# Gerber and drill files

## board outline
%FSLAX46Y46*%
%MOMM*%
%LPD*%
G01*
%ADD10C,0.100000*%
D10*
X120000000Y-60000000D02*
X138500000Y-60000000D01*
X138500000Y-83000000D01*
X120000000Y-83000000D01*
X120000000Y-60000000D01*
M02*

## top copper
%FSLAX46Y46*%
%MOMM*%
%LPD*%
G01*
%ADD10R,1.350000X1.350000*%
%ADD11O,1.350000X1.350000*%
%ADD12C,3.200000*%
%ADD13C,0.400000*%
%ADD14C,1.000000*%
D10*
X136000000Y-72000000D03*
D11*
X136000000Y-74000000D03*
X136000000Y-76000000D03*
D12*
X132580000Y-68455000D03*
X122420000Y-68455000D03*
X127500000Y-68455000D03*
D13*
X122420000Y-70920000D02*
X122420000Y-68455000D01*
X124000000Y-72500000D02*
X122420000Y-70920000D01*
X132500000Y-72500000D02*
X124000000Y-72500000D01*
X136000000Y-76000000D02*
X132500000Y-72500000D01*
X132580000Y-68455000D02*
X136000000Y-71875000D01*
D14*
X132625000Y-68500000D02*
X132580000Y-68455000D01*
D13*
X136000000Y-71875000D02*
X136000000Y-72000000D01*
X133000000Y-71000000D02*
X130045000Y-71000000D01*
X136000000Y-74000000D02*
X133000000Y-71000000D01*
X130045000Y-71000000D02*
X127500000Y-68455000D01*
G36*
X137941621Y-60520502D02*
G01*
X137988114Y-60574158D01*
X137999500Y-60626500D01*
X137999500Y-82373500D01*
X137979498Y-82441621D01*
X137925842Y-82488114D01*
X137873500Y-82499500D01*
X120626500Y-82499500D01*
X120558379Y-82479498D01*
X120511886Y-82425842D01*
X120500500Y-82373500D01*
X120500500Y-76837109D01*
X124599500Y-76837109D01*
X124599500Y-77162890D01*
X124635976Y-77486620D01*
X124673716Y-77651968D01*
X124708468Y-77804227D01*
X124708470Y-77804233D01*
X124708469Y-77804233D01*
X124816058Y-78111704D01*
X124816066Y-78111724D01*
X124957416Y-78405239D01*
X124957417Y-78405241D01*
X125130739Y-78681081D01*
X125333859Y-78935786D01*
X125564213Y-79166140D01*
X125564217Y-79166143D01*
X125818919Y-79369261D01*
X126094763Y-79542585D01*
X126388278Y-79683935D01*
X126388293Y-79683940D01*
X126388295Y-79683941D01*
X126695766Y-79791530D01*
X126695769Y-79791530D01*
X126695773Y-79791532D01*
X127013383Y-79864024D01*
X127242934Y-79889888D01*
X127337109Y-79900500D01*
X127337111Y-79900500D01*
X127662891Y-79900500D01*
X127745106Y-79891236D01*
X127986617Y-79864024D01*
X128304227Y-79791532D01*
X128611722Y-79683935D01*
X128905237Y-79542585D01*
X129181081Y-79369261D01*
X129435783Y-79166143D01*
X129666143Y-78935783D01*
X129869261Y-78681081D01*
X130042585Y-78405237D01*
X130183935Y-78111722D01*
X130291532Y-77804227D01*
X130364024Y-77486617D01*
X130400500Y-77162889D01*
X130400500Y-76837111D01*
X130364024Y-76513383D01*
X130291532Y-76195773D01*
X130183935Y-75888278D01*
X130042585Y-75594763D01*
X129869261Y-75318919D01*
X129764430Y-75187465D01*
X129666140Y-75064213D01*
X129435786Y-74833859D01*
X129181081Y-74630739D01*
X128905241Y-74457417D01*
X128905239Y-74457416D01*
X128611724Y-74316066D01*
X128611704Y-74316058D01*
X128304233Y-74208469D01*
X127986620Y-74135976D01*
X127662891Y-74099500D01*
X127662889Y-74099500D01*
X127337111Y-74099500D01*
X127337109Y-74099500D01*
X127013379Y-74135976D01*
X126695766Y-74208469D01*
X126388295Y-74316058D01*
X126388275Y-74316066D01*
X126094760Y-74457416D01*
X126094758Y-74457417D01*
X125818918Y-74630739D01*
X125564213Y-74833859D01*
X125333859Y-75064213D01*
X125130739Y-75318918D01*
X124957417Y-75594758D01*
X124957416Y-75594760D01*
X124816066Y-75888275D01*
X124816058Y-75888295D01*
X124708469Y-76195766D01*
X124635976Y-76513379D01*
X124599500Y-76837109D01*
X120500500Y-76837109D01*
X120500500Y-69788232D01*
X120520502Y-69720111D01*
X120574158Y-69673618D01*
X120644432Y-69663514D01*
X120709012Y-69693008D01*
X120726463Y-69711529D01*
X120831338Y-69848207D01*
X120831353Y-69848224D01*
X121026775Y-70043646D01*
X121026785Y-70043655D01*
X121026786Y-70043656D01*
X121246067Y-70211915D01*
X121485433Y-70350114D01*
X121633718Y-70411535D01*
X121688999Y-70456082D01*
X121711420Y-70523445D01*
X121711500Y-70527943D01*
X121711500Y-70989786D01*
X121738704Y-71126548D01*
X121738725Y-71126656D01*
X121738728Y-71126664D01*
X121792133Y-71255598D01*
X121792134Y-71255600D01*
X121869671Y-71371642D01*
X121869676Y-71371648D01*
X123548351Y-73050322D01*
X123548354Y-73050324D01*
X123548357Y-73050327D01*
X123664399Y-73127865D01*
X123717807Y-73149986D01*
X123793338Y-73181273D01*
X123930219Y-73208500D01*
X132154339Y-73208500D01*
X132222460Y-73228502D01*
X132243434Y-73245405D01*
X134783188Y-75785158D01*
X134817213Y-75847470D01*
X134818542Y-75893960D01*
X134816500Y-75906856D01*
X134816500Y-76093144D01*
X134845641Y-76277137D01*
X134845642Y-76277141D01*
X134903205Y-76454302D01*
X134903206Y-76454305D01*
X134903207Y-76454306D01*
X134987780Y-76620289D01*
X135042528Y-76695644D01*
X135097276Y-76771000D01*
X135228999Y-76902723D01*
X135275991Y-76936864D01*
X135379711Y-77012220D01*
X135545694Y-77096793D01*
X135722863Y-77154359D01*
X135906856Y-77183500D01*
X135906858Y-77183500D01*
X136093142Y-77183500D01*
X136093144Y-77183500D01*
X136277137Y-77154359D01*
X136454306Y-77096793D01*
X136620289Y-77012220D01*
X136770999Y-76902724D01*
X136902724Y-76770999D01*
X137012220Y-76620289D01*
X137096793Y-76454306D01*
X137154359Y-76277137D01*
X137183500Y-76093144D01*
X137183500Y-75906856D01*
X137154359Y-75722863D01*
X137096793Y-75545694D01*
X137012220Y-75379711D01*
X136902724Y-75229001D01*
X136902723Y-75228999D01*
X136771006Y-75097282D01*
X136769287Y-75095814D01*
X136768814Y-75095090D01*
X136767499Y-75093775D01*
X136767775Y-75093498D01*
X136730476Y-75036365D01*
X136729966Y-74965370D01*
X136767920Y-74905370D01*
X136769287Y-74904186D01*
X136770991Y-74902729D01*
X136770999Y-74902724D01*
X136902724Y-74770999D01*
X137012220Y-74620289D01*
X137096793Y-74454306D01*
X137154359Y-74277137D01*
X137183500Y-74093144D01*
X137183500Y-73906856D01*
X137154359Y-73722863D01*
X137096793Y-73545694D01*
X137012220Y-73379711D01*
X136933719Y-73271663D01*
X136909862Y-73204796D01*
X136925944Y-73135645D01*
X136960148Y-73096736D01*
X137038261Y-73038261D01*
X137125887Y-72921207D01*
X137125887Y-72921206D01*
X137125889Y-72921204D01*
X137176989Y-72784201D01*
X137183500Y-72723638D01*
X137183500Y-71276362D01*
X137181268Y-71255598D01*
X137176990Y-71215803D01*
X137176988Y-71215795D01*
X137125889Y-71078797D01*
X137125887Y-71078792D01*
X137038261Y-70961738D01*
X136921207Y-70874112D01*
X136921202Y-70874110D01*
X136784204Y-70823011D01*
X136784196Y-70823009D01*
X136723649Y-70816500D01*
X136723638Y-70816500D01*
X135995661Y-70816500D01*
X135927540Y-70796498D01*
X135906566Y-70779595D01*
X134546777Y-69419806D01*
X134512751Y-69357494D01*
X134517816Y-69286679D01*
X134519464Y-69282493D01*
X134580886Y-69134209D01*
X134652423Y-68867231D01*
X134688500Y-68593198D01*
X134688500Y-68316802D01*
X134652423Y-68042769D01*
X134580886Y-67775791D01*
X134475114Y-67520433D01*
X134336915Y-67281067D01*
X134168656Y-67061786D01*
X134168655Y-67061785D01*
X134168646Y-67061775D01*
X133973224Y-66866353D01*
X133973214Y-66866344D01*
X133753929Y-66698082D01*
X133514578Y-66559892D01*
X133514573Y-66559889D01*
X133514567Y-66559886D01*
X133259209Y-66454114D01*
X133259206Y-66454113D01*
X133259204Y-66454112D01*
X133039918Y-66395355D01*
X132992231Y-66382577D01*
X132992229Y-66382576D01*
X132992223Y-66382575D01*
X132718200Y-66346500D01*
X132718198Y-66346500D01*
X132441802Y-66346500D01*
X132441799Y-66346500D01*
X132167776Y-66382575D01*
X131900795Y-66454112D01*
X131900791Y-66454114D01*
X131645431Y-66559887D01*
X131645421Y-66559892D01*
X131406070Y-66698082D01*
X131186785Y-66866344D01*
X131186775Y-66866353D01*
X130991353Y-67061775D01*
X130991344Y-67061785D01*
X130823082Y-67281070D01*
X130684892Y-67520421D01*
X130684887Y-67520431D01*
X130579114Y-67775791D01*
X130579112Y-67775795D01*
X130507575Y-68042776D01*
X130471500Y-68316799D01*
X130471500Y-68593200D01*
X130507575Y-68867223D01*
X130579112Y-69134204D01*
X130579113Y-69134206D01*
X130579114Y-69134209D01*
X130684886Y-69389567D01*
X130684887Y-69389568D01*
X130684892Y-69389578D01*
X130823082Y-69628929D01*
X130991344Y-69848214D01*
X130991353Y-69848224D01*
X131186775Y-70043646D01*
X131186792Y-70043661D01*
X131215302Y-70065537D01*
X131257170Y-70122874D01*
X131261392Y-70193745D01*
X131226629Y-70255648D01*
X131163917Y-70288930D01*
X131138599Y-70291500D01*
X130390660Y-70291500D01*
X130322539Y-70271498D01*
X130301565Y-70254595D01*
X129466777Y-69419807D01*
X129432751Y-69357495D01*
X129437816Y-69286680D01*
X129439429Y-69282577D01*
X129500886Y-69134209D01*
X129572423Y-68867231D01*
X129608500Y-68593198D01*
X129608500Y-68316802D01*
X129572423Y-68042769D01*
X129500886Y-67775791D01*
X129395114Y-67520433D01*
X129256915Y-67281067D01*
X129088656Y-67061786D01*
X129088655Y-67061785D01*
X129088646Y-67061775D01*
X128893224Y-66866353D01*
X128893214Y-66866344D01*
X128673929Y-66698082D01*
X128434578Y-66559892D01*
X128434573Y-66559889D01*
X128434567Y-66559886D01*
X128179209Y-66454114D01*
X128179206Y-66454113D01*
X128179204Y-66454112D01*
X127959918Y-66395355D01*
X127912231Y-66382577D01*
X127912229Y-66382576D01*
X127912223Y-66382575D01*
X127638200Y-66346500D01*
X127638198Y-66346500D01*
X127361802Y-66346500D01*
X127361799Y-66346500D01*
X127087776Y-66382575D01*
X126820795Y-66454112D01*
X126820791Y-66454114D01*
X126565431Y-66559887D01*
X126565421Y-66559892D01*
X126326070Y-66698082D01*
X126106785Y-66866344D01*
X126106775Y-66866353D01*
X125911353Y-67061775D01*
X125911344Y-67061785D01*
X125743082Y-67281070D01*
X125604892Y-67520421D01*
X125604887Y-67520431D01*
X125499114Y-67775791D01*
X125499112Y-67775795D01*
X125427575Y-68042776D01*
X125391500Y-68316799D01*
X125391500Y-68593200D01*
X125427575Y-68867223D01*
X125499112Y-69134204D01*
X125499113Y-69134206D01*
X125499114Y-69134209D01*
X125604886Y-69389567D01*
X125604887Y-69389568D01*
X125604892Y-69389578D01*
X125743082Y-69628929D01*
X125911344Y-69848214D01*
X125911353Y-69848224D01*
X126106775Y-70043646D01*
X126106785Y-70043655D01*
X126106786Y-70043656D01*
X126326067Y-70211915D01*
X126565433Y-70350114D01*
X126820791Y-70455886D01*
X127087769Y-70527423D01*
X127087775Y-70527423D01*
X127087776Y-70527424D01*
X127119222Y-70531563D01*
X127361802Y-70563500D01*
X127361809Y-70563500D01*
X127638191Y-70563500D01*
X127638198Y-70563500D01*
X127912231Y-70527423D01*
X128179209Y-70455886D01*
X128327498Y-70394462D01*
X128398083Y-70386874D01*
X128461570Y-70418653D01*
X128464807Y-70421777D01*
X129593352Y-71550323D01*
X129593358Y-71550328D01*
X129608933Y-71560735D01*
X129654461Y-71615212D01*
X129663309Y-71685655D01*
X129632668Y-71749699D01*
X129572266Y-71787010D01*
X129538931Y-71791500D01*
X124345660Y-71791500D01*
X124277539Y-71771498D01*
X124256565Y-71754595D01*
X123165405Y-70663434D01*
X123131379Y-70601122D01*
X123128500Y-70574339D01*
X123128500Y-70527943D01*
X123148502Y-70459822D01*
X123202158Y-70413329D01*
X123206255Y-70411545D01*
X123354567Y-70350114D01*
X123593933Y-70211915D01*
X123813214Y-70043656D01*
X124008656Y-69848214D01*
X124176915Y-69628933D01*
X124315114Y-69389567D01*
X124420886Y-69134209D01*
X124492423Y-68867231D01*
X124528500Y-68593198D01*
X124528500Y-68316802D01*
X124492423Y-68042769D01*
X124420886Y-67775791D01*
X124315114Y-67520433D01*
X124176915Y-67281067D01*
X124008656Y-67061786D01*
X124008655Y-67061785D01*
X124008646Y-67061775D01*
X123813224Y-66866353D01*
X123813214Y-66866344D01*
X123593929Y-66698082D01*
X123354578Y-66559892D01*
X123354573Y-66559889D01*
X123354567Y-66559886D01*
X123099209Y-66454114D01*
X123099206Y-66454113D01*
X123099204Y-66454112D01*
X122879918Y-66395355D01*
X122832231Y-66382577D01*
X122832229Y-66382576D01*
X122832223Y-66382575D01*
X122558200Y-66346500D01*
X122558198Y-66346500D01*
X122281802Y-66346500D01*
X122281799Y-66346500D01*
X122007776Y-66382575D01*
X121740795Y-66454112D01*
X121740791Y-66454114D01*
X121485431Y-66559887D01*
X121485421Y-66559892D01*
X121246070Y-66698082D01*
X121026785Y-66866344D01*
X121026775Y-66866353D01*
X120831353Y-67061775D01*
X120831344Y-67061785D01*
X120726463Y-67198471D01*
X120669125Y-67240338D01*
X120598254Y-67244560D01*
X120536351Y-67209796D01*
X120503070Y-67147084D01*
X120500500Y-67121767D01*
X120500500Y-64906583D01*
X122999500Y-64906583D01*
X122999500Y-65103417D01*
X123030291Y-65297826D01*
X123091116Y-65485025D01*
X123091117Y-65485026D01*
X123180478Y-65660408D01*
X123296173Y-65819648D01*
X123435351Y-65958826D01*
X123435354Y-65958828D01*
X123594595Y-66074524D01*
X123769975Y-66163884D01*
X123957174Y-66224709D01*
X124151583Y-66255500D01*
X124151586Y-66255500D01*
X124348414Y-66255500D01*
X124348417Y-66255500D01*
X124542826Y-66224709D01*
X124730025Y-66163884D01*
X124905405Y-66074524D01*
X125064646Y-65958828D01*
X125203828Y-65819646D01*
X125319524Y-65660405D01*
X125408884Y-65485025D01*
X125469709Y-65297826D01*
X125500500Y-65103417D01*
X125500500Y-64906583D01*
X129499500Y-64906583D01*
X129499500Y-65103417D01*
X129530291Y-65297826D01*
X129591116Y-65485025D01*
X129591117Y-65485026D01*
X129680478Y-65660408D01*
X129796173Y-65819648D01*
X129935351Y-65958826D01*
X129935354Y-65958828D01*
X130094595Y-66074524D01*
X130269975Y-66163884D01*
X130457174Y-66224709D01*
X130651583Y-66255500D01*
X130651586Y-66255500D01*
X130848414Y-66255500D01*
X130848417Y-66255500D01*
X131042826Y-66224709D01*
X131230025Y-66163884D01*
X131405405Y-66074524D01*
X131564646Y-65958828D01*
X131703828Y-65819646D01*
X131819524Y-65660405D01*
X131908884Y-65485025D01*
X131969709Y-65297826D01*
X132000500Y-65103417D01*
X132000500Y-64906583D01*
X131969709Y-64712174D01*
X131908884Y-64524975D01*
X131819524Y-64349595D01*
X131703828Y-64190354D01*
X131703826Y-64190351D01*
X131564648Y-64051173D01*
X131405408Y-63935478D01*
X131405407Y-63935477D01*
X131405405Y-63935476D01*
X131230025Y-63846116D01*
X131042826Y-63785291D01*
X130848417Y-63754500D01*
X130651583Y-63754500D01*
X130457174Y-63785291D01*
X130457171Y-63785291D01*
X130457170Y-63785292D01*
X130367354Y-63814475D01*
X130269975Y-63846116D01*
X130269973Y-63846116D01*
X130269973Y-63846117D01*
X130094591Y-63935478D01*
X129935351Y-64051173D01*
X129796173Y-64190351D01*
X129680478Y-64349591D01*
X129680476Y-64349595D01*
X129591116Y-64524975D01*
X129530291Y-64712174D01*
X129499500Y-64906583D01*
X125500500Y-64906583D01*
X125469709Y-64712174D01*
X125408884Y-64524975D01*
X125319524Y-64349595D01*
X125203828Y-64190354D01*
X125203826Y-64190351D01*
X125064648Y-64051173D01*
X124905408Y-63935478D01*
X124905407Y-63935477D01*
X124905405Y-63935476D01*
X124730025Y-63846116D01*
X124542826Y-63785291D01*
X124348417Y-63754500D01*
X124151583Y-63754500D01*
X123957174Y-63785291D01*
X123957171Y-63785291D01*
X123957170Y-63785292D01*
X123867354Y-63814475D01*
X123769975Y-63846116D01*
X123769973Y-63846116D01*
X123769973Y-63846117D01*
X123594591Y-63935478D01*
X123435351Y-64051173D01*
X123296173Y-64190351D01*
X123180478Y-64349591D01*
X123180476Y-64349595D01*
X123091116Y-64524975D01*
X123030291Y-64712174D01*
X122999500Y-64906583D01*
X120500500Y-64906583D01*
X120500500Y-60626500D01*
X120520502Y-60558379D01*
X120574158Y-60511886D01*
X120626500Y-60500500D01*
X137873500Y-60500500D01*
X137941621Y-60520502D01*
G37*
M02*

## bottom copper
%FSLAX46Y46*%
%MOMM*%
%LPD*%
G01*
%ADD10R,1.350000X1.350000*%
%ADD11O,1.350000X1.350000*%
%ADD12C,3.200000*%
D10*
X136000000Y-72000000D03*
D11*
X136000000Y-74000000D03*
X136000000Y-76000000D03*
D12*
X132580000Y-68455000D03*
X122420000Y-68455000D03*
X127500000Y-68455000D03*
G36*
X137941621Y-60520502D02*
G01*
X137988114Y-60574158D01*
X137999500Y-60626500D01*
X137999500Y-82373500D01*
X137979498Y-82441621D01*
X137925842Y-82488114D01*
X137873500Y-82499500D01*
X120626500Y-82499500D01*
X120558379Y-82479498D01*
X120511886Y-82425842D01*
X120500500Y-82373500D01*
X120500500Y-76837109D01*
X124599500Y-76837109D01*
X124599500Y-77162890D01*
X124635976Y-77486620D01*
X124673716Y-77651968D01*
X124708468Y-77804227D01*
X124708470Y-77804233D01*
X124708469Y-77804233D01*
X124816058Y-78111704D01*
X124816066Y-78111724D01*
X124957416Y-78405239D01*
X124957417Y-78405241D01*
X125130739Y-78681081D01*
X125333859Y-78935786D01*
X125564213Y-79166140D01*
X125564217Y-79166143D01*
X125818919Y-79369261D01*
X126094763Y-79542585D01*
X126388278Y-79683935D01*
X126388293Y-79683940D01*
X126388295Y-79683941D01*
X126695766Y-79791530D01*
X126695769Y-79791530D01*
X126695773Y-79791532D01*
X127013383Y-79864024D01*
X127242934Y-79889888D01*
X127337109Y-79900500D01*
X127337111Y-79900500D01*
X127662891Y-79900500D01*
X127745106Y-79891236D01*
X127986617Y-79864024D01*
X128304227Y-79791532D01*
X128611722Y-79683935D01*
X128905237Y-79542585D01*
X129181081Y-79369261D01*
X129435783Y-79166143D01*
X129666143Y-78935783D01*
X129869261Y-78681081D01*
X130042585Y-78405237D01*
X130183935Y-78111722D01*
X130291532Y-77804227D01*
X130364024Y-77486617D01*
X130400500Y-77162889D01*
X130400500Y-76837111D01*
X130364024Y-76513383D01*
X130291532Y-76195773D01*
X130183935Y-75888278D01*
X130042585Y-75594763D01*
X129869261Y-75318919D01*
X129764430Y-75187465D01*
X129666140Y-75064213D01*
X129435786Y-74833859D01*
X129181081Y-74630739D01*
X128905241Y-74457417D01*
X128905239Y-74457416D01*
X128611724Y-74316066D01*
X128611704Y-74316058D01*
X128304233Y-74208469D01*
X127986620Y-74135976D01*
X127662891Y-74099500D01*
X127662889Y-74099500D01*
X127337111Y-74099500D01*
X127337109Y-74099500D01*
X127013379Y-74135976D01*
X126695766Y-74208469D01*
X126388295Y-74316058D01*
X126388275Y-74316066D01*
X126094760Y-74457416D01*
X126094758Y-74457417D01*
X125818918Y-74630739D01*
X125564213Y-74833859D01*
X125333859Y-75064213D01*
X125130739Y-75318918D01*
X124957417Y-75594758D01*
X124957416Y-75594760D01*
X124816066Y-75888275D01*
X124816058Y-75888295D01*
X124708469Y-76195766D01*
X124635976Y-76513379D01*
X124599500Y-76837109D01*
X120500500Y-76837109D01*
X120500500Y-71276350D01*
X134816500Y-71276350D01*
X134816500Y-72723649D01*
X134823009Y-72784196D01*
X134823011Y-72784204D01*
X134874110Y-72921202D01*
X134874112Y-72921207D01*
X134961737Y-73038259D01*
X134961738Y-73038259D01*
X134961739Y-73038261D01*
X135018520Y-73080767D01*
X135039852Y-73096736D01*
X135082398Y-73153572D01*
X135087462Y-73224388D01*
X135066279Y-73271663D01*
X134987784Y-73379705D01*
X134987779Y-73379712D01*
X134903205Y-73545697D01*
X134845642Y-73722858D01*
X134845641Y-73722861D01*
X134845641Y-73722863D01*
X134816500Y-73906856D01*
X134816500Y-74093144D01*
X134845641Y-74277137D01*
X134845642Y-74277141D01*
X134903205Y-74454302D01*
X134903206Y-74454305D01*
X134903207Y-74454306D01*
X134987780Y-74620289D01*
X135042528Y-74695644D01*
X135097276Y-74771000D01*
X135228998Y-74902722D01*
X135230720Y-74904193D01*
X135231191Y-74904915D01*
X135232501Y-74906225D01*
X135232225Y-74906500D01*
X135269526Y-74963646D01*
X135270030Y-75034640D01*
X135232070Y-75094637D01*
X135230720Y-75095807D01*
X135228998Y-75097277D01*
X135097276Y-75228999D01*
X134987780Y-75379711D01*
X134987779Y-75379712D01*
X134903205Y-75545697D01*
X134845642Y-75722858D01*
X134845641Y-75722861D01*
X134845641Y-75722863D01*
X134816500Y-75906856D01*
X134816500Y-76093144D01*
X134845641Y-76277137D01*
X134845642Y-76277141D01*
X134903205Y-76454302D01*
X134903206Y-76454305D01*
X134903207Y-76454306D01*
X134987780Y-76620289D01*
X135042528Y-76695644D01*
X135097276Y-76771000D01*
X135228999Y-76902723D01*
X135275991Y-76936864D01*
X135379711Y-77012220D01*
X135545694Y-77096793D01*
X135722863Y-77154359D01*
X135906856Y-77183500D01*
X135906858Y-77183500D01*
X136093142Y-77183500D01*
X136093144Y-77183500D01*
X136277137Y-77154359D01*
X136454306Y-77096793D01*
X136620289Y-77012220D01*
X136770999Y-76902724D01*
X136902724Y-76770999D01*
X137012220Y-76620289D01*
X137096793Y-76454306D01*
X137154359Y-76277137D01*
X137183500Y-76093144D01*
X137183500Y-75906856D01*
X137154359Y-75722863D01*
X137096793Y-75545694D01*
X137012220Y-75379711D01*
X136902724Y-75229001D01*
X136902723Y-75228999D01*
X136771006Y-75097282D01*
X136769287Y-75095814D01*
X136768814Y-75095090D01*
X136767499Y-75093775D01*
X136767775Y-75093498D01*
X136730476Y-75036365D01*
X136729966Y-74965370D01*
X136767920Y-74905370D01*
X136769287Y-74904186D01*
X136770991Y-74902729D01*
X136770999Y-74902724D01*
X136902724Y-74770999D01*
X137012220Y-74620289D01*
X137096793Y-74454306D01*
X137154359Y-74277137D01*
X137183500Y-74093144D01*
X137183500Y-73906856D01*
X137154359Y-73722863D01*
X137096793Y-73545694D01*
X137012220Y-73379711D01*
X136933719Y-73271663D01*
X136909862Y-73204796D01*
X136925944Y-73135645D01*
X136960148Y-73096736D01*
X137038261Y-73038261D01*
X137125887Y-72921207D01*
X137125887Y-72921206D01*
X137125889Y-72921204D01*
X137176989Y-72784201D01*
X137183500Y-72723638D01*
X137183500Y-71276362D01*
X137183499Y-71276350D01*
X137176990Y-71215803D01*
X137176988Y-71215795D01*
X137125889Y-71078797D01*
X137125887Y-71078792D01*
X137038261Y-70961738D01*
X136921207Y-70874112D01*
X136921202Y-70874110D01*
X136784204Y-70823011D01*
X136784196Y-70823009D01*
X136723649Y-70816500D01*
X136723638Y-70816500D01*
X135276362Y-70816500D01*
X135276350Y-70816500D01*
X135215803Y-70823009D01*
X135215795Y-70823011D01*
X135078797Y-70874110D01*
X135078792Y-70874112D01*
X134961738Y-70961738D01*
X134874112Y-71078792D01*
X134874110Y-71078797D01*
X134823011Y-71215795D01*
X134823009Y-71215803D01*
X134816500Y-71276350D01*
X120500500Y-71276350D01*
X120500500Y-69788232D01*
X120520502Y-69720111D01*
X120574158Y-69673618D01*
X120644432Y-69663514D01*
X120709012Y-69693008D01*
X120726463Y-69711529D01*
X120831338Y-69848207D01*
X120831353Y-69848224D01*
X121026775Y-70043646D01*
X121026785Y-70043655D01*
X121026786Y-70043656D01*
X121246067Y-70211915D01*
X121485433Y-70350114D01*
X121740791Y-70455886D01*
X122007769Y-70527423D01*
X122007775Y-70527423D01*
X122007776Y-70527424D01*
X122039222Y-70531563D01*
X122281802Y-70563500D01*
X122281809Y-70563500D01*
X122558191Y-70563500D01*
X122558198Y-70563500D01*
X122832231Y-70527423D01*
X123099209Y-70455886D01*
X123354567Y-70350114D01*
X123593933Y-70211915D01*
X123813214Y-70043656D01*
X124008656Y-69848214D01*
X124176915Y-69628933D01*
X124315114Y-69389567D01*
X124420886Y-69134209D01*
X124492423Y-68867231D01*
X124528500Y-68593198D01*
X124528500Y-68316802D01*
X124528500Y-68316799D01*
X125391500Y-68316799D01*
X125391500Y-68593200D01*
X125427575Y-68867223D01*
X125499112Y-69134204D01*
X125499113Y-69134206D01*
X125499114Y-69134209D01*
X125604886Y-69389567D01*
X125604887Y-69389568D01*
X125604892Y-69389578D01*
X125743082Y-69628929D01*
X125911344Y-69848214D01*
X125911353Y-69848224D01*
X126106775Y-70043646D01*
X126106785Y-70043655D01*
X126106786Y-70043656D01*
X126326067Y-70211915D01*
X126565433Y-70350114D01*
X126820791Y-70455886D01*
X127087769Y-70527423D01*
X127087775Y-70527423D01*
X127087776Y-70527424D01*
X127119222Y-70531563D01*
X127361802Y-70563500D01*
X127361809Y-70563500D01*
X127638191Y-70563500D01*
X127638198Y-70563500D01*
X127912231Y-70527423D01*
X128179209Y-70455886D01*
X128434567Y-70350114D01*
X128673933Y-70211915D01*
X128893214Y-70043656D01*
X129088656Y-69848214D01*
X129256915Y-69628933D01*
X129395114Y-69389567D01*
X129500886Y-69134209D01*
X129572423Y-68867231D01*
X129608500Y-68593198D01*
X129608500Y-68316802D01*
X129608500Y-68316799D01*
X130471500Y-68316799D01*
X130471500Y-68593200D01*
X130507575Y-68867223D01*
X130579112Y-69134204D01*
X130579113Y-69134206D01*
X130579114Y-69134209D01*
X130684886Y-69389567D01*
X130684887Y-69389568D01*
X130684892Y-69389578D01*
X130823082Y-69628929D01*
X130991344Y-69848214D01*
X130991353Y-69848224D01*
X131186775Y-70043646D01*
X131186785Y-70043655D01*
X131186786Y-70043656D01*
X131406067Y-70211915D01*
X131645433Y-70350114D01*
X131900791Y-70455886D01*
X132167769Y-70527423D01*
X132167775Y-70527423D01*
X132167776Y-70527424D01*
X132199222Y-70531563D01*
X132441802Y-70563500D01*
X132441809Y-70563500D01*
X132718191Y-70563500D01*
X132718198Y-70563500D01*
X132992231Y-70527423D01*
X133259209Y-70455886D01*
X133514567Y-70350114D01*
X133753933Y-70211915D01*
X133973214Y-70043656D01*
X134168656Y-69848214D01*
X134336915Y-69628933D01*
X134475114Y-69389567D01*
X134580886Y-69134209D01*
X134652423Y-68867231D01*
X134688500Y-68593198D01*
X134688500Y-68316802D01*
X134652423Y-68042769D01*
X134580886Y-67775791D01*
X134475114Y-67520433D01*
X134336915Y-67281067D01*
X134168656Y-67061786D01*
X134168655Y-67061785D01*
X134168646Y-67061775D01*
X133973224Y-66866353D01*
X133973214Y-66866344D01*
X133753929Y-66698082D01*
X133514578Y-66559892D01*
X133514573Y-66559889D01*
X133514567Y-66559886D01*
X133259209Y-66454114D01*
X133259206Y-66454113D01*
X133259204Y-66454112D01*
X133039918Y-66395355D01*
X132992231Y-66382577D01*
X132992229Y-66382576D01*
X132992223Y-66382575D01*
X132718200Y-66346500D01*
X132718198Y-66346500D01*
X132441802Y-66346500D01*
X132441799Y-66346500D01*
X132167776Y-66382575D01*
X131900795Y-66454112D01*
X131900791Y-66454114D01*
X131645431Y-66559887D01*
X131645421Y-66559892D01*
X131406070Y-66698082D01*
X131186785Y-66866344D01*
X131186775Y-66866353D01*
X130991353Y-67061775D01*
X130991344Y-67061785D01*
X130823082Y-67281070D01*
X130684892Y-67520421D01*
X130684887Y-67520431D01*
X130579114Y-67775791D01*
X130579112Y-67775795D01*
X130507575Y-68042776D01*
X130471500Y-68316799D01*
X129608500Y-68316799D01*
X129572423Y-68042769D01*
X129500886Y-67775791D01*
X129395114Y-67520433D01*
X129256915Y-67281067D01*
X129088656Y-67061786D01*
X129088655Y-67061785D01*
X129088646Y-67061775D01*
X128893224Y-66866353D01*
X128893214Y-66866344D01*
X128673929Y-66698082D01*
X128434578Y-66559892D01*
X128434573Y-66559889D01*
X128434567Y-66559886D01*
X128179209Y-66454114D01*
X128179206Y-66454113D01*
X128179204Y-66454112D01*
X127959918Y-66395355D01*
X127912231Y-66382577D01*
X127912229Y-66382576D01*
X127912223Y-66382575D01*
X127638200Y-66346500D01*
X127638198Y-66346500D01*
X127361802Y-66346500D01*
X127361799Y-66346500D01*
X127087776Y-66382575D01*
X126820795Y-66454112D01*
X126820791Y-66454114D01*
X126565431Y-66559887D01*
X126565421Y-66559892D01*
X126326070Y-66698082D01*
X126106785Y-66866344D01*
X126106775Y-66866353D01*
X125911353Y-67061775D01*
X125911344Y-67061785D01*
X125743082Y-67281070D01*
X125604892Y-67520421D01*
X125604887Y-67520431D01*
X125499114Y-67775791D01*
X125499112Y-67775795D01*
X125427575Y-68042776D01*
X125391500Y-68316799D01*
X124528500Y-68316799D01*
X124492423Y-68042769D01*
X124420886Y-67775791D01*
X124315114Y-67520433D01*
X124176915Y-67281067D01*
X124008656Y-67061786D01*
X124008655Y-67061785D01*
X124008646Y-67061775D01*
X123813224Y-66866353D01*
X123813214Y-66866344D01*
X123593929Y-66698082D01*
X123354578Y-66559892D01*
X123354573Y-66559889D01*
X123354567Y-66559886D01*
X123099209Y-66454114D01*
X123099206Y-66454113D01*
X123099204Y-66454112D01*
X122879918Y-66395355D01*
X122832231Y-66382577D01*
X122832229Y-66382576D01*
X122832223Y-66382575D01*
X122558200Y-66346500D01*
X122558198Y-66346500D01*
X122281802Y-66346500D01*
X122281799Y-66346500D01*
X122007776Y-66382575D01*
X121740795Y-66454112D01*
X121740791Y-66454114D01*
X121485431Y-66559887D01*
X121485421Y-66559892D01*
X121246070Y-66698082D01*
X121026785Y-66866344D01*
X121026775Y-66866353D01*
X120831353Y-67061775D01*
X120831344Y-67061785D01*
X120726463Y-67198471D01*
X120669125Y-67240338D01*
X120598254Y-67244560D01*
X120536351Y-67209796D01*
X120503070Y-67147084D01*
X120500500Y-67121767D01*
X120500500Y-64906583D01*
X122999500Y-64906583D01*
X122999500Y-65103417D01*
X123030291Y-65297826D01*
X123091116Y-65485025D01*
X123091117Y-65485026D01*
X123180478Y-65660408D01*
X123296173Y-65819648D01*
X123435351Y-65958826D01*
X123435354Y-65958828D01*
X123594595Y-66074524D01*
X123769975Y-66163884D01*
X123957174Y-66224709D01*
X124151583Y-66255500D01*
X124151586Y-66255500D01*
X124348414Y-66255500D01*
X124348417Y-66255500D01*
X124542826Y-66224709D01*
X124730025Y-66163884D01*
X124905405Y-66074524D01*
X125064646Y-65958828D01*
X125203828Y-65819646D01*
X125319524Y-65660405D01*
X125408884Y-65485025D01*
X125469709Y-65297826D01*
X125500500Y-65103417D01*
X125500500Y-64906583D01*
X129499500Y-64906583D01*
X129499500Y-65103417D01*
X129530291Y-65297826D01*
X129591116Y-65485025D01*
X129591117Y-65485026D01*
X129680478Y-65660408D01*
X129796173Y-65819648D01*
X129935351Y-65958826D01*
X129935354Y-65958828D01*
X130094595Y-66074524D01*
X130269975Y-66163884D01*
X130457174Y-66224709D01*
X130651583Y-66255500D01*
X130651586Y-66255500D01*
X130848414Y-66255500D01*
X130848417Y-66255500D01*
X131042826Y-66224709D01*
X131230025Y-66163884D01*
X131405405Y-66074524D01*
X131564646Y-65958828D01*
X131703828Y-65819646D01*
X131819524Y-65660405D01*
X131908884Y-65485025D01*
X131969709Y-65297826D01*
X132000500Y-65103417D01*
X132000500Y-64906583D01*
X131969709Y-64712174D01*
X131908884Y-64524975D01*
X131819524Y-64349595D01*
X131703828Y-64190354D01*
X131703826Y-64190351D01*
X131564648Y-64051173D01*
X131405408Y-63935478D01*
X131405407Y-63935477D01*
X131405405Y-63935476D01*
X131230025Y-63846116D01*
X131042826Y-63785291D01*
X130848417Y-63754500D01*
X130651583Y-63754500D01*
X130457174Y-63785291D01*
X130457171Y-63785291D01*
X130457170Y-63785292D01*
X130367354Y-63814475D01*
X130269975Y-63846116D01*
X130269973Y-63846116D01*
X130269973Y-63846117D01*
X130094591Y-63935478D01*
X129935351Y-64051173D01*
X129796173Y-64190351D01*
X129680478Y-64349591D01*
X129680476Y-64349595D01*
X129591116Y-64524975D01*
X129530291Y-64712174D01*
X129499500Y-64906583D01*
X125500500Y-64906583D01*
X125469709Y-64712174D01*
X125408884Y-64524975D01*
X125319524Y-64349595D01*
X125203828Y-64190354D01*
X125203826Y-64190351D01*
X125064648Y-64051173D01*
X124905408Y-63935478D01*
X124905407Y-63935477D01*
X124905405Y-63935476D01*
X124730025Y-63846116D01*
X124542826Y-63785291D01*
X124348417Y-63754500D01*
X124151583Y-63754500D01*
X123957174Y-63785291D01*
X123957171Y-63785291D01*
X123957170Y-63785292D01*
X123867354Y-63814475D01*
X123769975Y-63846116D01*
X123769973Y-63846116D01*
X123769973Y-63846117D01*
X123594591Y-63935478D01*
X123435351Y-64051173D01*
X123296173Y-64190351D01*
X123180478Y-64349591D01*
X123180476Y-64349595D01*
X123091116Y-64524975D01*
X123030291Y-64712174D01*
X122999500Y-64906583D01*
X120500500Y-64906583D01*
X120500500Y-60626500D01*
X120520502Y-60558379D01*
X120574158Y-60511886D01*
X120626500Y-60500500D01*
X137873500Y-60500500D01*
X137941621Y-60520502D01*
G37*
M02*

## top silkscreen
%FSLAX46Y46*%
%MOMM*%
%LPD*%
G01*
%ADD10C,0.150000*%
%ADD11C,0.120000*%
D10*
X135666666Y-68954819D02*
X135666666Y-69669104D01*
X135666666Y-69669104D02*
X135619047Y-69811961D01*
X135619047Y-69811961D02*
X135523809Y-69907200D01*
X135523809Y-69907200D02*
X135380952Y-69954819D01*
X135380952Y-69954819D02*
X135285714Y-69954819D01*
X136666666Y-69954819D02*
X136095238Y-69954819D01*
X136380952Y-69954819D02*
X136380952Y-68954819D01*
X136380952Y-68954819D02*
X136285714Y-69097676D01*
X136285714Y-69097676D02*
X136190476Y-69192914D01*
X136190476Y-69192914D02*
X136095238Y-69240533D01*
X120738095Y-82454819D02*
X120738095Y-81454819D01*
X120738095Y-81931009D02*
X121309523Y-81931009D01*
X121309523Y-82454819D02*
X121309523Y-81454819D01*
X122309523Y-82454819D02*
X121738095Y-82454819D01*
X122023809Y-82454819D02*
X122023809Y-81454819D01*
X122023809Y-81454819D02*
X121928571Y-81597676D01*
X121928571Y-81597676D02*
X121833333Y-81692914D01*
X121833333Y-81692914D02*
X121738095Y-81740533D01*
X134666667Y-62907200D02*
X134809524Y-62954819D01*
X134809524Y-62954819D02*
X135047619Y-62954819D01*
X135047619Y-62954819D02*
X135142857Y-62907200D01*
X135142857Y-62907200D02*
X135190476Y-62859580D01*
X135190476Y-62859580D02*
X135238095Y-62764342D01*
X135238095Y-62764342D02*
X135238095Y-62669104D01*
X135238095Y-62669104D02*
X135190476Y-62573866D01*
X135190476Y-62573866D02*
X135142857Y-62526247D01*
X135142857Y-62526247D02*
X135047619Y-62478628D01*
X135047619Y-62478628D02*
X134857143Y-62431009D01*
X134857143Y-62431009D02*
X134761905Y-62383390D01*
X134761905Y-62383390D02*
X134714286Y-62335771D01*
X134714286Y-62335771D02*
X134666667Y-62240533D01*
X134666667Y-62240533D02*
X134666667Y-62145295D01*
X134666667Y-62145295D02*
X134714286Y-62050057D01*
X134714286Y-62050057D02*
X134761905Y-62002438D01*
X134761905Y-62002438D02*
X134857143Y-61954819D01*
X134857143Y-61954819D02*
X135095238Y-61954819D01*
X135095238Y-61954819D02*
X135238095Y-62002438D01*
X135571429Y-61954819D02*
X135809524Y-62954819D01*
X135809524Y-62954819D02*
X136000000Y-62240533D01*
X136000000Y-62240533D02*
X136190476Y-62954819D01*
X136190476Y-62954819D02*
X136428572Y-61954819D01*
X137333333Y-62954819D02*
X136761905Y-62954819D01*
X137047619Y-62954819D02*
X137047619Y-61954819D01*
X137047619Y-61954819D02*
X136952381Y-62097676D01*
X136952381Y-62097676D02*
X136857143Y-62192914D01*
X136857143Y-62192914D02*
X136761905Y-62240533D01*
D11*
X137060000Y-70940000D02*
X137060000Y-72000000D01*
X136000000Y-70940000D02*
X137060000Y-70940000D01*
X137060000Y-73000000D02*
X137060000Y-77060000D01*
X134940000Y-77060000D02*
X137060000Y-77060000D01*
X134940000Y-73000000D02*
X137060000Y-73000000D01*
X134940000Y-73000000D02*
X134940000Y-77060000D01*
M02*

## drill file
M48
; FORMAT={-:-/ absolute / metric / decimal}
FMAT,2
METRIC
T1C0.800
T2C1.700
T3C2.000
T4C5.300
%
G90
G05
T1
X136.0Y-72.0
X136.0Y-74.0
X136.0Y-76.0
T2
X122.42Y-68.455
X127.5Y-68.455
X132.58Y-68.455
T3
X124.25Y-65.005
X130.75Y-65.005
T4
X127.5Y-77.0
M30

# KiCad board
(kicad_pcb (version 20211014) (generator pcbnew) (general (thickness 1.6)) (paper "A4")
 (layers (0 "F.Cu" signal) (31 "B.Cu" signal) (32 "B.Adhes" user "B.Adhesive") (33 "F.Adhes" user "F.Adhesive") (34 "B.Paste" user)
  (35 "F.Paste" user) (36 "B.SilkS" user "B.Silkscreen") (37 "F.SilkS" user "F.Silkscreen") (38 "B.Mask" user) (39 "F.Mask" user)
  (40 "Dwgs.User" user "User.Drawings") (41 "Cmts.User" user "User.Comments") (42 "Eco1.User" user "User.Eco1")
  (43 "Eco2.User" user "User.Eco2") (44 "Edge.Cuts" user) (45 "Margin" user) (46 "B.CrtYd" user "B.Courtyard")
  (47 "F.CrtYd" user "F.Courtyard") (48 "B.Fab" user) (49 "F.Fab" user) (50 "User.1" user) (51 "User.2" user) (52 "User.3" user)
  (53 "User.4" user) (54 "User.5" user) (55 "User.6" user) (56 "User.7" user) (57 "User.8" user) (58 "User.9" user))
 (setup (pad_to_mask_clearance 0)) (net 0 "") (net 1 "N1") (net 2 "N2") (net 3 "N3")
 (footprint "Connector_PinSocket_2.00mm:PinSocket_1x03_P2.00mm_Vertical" (layer "F.Cu") (at 136 72)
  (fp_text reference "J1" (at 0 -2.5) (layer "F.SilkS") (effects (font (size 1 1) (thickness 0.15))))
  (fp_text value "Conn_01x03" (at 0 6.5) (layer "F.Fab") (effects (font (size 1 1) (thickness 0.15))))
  (fp_line (start 1.06 -1.06) (end 1.06 0) (layer "F.SilkS") (width 0.12))
  (fp_line (start 0 -1.06) (end 1.06 -1.06) (layer "F.SilkS") (width 0.12))
  (fp_line (start 1.06 1) (end 1.06 5.06) (layer "F.SilkS") (width 0.12))
  (fp_line (start -1.06 5.06) (end 1.06 5.06) (layer "F.SilkS") (width 0.12))
  (fp_line (start -1.06 1) (end 1.06 1) (layer "F.SilkS") (width 0.12))
  (fp_line (start -1.06 1) (end -1.06 5.06) (layer "F.SilkS") (width 0.12))
  (pad "1" thru_hole rect (at 0 0) (size 1.35 1.35) (drill 0.8) (layers *.Cu *.Mask) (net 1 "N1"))
  (pad "2" thru_hole oval (at 0 2) (size 1.35 1.35) (drill 0.8) (layers *.Cu *.Mask) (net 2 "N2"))
  (pad "3" thru_hole oval (at 0 4) (size 1.35 1.35) (drill 0.8) (layers *.Cu *.Mask) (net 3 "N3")))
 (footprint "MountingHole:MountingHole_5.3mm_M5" (layer "F.Cu") (at 127.5 77)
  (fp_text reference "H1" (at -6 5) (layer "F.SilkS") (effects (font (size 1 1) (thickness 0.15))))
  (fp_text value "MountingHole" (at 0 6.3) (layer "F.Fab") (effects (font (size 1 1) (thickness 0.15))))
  (pad "" np_thru_hole circle (at 0 0) (size 5.3 5.3) (drill 5.3) (layers *.Cu *.Mask)))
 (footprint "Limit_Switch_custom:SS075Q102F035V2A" (layer "F.Cu") (at 127.5 68.455)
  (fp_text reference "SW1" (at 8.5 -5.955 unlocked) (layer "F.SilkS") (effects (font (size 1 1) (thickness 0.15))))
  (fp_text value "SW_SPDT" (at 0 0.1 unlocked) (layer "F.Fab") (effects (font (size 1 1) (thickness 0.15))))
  (pad "" np_thru_hole circle (at 3.25 -3.45) (size 2 2) (drill 2) (layers F&B.Cu *.Mask))
  (pad "" np_thru_hole circle (at -3.25 -3.45) (size 2 2) (drill 2) (layers F&B.Cu *.Mask))
  (pad "1" thru_hole circle (at 5.08 0) (size 3.2 3.2) (drill 1.7) (layers *.Cu *.Mask) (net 1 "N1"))
  (pad "2" thru_hole circle (at -5.08 0) (size 3.2 3.2) (drill 1.7) (layers *.Cu *.Mask) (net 3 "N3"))
  (pad "3" thru_hole circle (at 0 0) (size 3.2 3.2) (drill 1.7) (layers *.Cu *.Mask) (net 2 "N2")))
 (gr_rect (start 120 60) (end 138.5 83) (layer "Edge.Cuts") (width 0.1) (fill none))
 (segment (start 122.42 70.92) (end 122.42 68.455) (width 0.4) (layer "F.Cu") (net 3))
 (segment (start 124 72.5) (end 122.42 70.92) (width 0.4) (layer "F.Cu") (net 3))
 (segment (start 132.5 72.5) (end 124 72.5) (width 0.4) (layer "F.Cu") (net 3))
 (segment (start 136 76) (end 132.5 72.5) (width 0.4) (layer "F.Cu") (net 3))
 (segment (start 132.58 68.455) (end 136 71.875) (width 0.4) (layer "F.Cu") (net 1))
 (segment (start 132.625 68.5) (end 132.58 68.455) (width 1) (layer "F.Cu") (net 1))
 (segment (start 136 71.875) (end 136 72) (width 0.4) (layer "F.Cu") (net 1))
 (segment (start 133 71) (end 130.045 71) (width 0.4) (layer "F.Cu") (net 2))
 (segment (start 136 74) (end 133 71) (width 0.4) (layer "F.Cu") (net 2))
 (segment (start 130.045 71) (end 127.5 68.455) (width 0.4) (layer "F.Cu") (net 2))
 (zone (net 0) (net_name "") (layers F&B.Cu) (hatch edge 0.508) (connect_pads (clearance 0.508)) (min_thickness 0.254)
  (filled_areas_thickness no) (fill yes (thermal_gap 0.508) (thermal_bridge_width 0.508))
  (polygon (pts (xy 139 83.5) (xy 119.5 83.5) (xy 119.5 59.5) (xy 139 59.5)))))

